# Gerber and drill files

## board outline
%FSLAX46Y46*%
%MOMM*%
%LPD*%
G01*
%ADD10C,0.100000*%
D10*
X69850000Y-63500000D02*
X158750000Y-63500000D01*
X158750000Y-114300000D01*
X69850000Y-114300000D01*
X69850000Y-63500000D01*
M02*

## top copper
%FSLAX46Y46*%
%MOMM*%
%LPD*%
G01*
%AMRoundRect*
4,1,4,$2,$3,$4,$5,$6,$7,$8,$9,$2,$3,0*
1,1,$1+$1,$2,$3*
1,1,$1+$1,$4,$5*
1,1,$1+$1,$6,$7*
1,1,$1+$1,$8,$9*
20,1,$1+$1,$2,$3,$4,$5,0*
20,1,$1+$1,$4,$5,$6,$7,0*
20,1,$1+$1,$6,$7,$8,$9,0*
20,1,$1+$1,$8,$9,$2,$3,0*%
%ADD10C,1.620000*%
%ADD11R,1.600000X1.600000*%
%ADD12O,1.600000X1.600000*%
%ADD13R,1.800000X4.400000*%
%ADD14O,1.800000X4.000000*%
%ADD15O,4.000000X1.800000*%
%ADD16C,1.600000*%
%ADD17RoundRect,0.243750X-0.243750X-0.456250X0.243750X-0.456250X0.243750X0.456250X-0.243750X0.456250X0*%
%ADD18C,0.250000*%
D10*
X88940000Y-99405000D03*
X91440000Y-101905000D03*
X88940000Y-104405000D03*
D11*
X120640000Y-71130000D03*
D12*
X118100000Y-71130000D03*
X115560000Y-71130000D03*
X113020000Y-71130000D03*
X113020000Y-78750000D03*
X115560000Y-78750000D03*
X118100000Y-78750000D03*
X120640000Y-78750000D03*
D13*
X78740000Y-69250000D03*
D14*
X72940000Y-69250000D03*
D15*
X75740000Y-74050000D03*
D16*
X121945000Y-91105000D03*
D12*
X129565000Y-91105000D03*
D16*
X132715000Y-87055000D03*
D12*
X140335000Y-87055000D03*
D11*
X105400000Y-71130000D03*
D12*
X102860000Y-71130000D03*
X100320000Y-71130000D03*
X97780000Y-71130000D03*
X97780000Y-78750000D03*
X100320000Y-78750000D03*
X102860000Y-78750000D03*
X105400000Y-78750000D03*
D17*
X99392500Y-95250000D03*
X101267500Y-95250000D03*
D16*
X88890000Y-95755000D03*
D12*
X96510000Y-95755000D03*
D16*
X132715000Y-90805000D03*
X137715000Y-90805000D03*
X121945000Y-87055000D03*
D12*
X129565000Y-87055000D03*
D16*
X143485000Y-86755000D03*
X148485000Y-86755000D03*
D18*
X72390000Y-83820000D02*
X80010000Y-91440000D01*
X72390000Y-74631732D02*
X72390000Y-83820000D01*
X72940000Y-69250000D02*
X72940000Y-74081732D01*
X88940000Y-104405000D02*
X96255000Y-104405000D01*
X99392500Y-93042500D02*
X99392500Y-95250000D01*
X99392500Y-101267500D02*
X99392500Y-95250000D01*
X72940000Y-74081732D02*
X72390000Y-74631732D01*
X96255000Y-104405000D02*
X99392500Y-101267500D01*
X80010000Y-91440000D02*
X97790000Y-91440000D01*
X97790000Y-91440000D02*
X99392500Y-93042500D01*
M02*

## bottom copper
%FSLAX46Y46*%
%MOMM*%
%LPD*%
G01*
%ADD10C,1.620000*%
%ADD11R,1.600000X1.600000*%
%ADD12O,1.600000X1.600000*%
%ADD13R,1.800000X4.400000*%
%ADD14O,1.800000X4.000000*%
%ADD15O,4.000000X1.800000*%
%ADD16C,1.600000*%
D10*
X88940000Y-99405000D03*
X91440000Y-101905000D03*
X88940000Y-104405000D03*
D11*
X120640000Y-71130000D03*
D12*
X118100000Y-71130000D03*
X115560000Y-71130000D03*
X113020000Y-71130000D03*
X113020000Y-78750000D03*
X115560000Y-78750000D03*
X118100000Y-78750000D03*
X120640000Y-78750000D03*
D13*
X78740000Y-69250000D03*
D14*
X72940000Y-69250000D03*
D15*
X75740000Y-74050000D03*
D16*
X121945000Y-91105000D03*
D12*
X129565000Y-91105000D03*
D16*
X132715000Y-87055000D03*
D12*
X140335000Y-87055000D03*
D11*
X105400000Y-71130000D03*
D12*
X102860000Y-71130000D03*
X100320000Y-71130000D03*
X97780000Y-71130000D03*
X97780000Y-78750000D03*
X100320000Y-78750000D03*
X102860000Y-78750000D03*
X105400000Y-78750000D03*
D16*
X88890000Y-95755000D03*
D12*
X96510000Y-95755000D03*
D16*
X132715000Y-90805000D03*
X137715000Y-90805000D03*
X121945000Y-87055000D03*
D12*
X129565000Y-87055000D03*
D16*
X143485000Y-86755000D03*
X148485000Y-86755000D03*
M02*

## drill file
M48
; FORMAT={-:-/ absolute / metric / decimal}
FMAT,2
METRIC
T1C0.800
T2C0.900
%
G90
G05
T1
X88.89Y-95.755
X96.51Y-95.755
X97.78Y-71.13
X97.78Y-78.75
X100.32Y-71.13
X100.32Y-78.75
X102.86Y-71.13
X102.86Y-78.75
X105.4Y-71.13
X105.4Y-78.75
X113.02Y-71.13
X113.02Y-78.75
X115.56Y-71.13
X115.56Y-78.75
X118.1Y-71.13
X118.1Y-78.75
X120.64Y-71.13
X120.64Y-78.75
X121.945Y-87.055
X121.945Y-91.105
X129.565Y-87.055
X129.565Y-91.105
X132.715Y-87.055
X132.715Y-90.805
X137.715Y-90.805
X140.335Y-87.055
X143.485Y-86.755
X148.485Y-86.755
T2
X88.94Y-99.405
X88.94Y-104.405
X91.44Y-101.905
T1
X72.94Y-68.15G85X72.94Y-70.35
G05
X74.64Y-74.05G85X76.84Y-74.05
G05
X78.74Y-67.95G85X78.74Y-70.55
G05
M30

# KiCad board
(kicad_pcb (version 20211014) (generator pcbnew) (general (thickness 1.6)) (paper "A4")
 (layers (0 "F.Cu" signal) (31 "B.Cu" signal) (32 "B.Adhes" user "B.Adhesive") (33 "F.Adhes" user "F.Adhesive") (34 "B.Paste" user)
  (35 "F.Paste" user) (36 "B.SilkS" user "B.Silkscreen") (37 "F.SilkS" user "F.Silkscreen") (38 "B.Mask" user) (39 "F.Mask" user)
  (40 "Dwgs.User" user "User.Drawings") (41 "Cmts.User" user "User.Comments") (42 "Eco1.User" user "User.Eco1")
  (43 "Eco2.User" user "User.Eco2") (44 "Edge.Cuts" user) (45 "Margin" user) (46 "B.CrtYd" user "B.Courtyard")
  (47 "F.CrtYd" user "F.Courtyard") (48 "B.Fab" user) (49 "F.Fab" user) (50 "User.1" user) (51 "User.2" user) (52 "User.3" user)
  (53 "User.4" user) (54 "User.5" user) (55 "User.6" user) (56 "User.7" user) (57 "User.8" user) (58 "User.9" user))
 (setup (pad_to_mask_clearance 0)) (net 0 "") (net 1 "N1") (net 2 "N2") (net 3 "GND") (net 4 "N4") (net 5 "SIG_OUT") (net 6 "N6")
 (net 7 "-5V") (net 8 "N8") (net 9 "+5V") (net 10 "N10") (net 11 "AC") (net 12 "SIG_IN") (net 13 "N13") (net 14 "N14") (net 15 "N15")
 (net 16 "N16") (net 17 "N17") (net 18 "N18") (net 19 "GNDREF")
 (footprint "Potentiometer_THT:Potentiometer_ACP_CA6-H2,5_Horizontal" (layer "F.Cu") (at 88.94 99.405)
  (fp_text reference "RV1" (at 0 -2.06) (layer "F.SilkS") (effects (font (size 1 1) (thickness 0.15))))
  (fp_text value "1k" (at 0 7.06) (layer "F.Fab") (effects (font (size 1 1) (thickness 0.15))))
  (pad "1" thru_hole circle locked (at 0 0) (size 1.62 1.62) (drill 0.9) (layers *.Cu *.Mask) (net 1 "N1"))
  (pad "2" thru_hole circle locked (at 2.5 2.5) (size 1.62 1.62) (drill 0.9) (layers *.Cu *.Mask) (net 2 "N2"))
  (pad "3" thru_hole circle locked (at 0 5) (size 1.62 1.62) (drill 0.9) (layers *.Cu *.Mask) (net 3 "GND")))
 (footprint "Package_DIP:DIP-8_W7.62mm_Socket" (layer "F.Cu") (at 120.64 71.13 -90)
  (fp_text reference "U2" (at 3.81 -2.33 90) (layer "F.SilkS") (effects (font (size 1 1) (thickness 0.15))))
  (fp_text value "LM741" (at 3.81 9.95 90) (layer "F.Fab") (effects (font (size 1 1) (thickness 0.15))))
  (pad "1" thru_hole rect (at 0 0 270) (size 1.6 1.6) (drill 0.8) (layers *.Cu *.Mask) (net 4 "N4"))
  (pad "2" thru_hole oval (at 0 2.54 270) (size 1.6 1.6) (drill 0.8) (layers *.Cu *.Mask) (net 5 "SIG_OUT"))
  (pad "3" thru_hole oval (at 0 5.08 270) (size 1.6 1.6) (drill 0.8) (layers *.Cu *.Mask) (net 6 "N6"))
  (pad "4" thru_hole oval (at 0 7.62 270) (size 1.6 1.6) (drill 0.8) (layers *.Cu *.Mask) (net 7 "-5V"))
  (pad "5" thru_hole oval (at 7.62 7.62 270) (size 1.6 1.6) (drill 0.8) (layers *.Cu *.Mask) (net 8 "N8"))
  (pad "6" thru_hole oval (at 7.62 5.08 270) (size 1.6 1.6) (drill 0.8) (layers *.Cu *.Mask) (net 5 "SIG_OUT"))
  (pad "7" thru_hole oval (at 7.62 2.54 270) (size 1.6 1.6) (drill 0.8) (layers *.Cu *.Mask) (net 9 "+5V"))
  (pad "8" thru_hole oval (at 7.62 0 270) (size 1.6 1.6) (drill 0.8) (layers *.Cu *.Mask) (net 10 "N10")))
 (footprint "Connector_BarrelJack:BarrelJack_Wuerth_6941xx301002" (layer "F.Cu") (at 78.74 69.25 -90)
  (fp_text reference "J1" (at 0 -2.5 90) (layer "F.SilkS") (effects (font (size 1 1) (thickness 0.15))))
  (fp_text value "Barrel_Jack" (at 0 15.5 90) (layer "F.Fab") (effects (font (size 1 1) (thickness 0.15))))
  (pad "1" thru_hole rect locked (at 0 0 270) (size 4.4 1.8) (drill oval 3.4 0.8) (layers *.Cu *.Mask) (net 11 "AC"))
  (pad "2" thru_hole oval locked (at 0 5.8 270) (size 4 1.8) (drill oval 3 0.8) (layers *.Cu *.Mask) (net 3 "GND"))
  (pad "3" thru_hole oval locked (at 4.8 3) (size 4 1.8) (drill oval 3 0.8) (layers *.Cu *.Mask)))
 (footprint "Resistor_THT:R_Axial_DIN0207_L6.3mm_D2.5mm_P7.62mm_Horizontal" (layer "F.Cu") (at 121.945 91.105)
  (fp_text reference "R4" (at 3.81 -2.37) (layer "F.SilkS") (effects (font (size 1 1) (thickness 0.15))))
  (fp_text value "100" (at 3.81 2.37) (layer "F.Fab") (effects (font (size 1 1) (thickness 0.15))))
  (pad "1" thru_hole circle (at 0 0) (size 1.6 1.6) (drill 0.8) (layers *.Cu *.Mask) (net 2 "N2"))
  (pad "2" thru_hole oval (at 7.62 0) (size 1.6 1.6) (drill 0.8) (layers *.Cu *.Mask) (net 6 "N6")))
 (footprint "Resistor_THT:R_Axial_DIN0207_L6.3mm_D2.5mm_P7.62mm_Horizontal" (layer "F.Cu") (at 132.715 87.055)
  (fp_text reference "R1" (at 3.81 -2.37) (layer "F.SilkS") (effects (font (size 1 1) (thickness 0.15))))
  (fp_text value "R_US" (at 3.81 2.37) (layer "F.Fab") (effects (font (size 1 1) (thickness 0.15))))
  (pad "1" thru_hole circle (at 0 0) (size 1.6 1.6) (drill 0.8) (layers *.Cu *.Mask) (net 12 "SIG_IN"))
  (pad "2" thru_hole oval (at 7.62 0) (size 1.6 1.6) (drill 0.8) (layers *.Cu *.Mask) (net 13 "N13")))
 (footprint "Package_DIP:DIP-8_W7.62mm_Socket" (layer "F.Cu") (at 105.4 71.13 -90)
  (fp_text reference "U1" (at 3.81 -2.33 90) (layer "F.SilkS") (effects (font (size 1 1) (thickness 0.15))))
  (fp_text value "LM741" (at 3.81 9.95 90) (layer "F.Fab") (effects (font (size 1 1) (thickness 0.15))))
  (pad "1" thru_hole rect (at 0 0 270) (size 1.6 1.6) (drill 0.8) (layers *.Cu *.Mask) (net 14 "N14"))
  (pad "2" thru_hole oval (at 0 2.54 270) (size 1.6 1.6) (drill 0.8) (layers *.Cu *.Mask) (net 2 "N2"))
  (pad "3" thru_hole oval (at 0 5.08 270) (size 1.6 1.6) (drill 0.8) (layers *.Cu *.Mask) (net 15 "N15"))
  (pad "4" thru_hole oval (at 0 7.62 270) (size 1.6 1.6) (drill 0.8) (layers *.Cu *.Mask) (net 7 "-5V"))
  (pad "5" thru_hole oval (at 7.62 7.62 270) (size 1.6 1.6) (drill 0.8) (layers *.Cu *.Mask) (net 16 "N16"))
  (pad "6" thru_hole oval (at 7.62 5.08 270) (size 1.6 1.6) (drill 0.8) (layers *.Cu *.Mask) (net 6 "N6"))
  (pad "7" thru_hole oval (at 7.62 2.54 270) (size 1.6 1.6) (drill 0.8) (layers *.Cu *.Mask) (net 9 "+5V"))
  (pad "8" thru_hole oval (at 7.62 0 270) (size 1.6 1.6) (drill 0.8) (layers *.Cu *.Mask) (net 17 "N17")))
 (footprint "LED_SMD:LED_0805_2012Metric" (layer "F.Cu") (at 100.33 95.25)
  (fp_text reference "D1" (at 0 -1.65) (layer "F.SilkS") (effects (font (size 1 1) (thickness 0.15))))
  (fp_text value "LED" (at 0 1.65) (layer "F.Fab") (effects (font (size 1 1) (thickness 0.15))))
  (pad "1" smd roundrect locked (at -0.9375 0) (size 0.975 1.4) (layers "F.Cu" "F.Paste" "F.Mask") (roundrect_rratio 0.25) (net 3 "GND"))
  (pad "2" smd roundrect locked (at 0.9375 0) (size 0.975 1.4) (layers "F.Cu" "F.Paste" "F.Mask") (roundrect_rratio 0.25) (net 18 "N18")))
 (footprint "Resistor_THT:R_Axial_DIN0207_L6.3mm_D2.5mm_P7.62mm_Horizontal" (layer "F.Cu") (at 88.89 95.755)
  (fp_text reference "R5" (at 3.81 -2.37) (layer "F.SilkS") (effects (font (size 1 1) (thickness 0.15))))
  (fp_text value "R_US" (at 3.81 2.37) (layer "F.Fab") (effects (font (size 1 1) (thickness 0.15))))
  (pad "1" thru_hole circle locked (at 0 0) (size 1.6 1.6) (drill 0.8) (layers *.Cu *.Mask) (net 9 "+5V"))
  (pad "2" thru_hole oval locked (at 7.62 0) (size 1.6 1.6) (drill 0.8) (layers *.Cu *.Mask) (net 18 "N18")))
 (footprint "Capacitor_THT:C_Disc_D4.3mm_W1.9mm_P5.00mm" (layer "F.Cu") (at 132.715 90.805)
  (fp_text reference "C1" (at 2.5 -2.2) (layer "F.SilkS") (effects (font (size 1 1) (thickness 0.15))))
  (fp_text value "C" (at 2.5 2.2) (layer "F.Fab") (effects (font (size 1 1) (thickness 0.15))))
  (pad "1" thru_hole circle (at 0 0) (size 1.6 1.6) (drill 0.8) (layers *.Cu *.Mask) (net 15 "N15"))
  (pad "2" thru_hole circle (at 5 0) (size 1.6 1.6) (drill 0.8) (layers *.Cu *.Mask) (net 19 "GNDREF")))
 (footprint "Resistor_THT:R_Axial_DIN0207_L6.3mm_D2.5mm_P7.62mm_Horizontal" (layer "F.Cu") (at 121.945 87.055)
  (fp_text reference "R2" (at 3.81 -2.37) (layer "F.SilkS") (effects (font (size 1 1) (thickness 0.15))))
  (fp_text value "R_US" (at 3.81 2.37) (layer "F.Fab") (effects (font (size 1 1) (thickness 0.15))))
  (pad "1" thru_hole circle (at 0 0) (size 1.6 1.6) (drill 0.8) (layers *.Cu *.Mask) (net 13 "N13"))
  (pad "2" thru_hole oval (at 7.62 0) (size 1.6 1.6) (drill 0.8) (layers *.Cu *.Mask) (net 15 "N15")))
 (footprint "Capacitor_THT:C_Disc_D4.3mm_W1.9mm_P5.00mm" (layer "F.Cu") (at 143.485 86.755)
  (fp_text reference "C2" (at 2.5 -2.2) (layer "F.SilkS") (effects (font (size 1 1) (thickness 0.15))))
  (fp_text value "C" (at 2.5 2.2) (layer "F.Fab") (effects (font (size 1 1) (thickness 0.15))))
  (pad "1" thru_hole circle (at 0 0) (size 1.6 1.6) (drill 0.8) (layers *.Cu *.Mask) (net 13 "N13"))
  (pad "2" thru_hole circle (at 5 0) (size 1.6 1.6) (drill 0.8) (layers *.Cu *.Mask) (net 6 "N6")))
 (gr_rect (start 69.85 63.5) (end 158.75 114.3) (layer "Edge.Cuts") (width 0.1) (fill none))
 (segment (start 72.39 83.82) (end 80.01 91.44) (width 0.25) (layer "F.Cu") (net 3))
 (segment (start 72.39 74.631732) (end 72.39 83.82) (width 0.25) (layer "F.Cu") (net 3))
 (segment (start 72.94 69.25) (end 72.94 74.081732) (width 0.25) (layer "F.Cu") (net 3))
 (segment (start 88.94 104.405) (end 96.255 104.405) (width 0.25) (layer "F.Cu") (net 3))
 (segment (start 99.3925 93.0425) (end 99.3925 95.25) (width 0.25) (layer "F.Cu") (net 3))
 (segment (start 99.3925 101.2675) (end 99.3925 95.25) (width 0.25) (layer "F.Cu") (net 3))
 (segment (start 72.94 74.081732) (end 72.39 74.631732) (width 0.25) (layer "F.Cu") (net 3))
 (segment (start 96.255 104.405) (end 99.3925 101.2675) (width 0.25) (layer "F.Cu") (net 3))
 (segment (start 80.01 91.44) (end 97.79 91.44) (width 0.25) (layer "F.Cu") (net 3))
 (segment (start 97.79 91.44) (end 99.3925 93.0425) (width 0.25) (layer "F.Cu") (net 3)))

